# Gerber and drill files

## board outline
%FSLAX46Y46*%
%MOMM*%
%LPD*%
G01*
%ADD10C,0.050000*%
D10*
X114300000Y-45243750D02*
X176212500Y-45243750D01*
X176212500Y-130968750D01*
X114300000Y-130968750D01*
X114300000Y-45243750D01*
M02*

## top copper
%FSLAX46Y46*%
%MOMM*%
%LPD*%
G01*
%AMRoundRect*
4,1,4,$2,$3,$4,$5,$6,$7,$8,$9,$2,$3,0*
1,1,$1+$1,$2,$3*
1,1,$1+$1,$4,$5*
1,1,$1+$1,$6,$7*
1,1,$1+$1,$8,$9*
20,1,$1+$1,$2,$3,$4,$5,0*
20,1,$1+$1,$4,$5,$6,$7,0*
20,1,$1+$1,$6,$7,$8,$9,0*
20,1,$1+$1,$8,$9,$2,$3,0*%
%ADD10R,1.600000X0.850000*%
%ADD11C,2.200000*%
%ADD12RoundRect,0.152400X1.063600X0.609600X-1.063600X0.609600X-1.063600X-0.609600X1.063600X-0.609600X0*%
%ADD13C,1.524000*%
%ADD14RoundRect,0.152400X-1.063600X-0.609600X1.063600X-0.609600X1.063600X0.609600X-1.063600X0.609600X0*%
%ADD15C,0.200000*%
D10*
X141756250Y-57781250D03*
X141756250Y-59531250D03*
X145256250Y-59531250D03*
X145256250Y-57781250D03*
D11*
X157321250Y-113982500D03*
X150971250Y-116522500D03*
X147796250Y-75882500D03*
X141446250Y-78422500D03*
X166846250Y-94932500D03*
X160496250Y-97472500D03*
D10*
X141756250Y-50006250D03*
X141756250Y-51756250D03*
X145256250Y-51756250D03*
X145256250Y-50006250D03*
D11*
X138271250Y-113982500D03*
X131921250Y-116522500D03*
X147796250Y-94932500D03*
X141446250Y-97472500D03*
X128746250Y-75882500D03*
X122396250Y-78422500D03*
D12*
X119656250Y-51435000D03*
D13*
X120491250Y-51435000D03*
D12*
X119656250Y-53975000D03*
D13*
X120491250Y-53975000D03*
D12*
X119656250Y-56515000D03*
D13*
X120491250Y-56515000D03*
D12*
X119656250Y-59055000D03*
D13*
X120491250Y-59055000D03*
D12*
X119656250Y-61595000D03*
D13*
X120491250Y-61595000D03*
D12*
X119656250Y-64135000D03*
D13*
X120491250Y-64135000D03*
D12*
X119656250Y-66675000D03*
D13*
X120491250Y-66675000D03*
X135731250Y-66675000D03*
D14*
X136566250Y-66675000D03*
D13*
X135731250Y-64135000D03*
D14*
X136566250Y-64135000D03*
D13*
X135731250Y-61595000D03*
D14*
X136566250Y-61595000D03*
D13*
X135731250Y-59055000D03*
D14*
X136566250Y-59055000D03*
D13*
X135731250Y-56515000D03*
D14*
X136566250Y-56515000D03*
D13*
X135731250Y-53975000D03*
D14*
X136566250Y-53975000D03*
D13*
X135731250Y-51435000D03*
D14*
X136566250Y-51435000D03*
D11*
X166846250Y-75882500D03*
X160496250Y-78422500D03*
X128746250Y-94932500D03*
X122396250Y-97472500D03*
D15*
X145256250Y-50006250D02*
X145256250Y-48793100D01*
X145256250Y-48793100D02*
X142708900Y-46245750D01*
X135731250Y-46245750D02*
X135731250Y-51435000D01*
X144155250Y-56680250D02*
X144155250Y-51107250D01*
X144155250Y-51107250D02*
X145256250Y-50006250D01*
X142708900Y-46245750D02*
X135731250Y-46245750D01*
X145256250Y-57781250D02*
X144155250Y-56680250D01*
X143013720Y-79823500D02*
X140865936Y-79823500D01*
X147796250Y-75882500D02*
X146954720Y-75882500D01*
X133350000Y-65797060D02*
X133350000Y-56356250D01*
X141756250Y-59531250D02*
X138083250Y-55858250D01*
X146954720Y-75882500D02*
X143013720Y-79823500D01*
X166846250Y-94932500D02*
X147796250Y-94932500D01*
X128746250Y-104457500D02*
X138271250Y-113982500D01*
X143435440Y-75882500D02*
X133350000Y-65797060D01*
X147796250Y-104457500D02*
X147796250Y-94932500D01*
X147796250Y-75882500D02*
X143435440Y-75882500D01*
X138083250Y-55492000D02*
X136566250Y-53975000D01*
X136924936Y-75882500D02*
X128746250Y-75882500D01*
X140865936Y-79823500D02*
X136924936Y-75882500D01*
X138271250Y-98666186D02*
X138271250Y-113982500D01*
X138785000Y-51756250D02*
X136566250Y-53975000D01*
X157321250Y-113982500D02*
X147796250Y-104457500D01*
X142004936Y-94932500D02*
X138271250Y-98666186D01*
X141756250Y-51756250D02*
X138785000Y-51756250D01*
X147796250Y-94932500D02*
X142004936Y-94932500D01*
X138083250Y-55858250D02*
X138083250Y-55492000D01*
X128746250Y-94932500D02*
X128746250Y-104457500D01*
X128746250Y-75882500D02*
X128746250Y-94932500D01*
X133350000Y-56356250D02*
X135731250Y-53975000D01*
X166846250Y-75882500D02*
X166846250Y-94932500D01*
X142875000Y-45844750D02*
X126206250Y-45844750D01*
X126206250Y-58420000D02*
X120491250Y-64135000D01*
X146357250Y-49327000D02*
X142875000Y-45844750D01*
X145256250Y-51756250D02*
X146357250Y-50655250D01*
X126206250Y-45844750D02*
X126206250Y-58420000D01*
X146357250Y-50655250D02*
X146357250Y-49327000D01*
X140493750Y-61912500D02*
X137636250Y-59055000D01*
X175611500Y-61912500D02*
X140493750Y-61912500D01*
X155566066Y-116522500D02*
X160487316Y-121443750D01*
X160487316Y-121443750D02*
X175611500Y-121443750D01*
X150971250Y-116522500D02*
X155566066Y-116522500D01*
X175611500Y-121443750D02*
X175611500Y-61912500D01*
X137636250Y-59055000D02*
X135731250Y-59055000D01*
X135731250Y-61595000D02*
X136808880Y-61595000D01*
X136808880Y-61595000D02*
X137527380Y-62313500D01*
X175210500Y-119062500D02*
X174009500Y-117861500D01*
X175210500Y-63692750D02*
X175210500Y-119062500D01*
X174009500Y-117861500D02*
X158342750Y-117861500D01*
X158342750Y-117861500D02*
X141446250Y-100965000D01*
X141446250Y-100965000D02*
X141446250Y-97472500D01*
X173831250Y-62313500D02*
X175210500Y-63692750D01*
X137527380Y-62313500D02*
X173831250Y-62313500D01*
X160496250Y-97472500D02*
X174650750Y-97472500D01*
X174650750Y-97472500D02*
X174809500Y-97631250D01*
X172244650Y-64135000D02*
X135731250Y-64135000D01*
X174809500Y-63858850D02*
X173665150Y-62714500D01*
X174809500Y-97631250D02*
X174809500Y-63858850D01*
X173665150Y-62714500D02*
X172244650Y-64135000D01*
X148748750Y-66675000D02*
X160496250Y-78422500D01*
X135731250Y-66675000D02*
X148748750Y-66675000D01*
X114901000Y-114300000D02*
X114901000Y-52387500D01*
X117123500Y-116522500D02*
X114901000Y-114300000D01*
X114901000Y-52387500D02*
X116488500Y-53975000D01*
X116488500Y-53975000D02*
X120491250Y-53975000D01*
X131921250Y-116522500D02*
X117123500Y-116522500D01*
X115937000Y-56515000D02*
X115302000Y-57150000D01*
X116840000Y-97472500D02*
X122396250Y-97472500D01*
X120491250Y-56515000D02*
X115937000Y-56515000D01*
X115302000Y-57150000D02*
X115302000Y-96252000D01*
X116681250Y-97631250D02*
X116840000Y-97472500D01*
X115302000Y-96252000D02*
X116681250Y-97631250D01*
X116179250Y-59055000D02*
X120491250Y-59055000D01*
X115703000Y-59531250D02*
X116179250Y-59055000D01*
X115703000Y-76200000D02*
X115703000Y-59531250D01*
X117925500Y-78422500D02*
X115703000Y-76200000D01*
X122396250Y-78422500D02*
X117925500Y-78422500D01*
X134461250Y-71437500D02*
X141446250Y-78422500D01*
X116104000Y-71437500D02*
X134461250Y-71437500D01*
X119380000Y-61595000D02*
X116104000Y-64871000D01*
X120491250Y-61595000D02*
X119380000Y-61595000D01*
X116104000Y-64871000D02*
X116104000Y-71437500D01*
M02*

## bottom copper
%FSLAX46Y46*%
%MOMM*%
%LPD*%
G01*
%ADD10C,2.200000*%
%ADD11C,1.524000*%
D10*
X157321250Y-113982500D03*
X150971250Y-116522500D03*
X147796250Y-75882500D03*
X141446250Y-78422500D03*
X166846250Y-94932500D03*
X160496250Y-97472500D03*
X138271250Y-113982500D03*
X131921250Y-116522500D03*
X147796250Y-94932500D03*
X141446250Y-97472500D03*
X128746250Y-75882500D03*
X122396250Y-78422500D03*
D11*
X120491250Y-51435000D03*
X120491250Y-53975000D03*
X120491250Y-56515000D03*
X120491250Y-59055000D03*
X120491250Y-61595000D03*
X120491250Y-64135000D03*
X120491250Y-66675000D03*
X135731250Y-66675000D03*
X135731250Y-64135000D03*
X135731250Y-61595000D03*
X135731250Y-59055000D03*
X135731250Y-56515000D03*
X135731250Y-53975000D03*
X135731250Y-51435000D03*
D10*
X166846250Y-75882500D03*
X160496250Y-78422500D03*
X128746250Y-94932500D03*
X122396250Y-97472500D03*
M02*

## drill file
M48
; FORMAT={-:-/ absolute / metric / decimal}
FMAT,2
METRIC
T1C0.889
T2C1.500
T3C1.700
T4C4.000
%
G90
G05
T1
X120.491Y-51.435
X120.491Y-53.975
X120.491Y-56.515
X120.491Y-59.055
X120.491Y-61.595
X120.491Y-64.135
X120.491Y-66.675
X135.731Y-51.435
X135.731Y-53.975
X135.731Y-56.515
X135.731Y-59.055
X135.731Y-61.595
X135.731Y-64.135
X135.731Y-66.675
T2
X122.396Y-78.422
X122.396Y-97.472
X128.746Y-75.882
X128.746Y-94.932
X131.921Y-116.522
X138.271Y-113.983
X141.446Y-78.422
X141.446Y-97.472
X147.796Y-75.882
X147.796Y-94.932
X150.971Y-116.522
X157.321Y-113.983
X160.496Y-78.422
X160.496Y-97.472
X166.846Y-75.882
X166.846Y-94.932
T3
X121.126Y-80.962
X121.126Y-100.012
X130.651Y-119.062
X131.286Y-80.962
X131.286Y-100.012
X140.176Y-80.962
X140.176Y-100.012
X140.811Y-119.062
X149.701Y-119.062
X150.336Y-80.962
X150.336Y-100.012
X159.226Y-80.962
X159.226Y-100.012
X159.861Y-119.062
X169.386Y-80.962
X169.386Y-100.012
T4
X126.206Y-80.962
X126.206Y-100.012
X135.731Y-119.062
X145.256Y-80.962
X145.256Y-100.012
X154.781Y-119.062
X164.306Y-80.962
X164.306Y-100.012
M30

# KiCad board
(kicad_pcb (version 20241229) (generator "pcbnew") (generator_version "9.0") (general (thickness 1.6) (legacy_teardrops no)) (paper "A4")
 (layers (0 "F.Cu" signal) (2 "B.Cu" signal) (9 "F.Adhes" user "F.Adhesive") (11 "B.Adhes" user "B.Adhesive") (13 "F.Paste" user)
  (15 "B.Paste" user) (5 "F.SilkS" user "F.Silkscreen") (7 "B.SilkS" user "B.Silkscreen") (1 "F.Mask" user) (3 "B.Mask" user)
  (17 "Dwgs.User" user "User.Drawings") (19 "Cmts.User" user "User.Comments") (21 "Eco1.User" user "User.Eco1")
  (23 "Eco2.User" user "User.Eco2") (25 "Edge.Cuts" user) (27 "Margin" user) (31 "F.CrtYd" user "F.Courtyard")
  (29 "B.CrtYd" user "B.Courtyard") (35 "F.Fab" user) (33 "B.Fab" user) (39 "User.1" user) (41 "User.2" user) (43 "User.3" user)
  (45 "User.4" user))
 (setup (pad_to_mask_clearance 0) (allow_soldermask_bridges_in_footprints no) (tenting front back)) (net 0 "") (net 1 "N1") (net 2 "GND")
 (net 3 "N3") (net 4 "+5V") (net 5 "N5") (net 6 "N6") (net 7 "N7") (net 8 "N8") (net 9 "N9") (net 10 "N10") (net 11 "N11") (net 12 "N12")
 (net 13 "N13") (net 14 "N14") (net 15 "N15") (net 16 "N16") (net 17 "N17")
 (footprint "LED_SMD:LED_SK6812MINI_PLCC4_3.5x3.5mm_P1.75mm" (layer "F.Cu") (at 143.50625 58.65625)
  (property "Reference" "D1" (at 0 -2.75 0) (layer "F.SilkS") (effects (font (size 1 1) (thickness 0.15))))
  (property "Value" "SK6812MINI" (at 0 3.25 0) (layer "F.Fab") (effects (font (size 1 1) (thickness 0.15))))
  (pad "1" smd rect (at -1.75 -0.875) (size 1.6 0.85) (layers "F.Cu" "F.Mask" "F.Paste") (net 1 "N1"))
  (pad "2" smd rect (at -1.75 0.875) (size 1.6 0.85) (layers "F.Cu" "F.Mask" "F.Paste") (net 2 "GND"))
  (pad "3" smd rect (at 1.75 0.875) (size 1.6 0.85) (layers "F.Cu" "F.Mask" "F.Paste") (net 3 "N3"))
  (pad "4" smd rect (at 1.75 -0.875) (size 1.6 0.85) (layers "F.Cu" "F.Mask" "F.Paste") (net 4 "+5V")))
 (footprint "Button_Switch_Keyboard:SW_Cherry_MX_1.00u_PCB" (layer "F.Cu") (at 157.32125 113.9825)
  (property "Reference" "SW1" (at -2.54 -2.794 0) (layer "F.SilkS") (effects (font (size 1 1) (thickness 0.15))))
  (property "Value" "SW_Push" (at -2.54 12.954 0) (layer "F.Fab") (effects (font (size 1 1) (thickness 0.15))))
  (pad "" np_thru_hole circle (at -7.62 5.08) (size 1.7 1.7) (drill 1.7) (layers "*.Cu" "*.Mask"))
  (pad "" np_thru_hole circle (at -2.54 5.08) (size 4 4) (drill 4) (layers "*.Cu" "*.Mask"))
  (pad "" np_thru_hole circle (at 2.54 5.08) (size 1.7 1.7) (drill 1.7) (layers "*.Cu" "*.Mask"))
  (pad "1" thru_hole circle (at 0 0) (size 2.2 2.2) (drill 1.5) (layers "*.Cu" "*.Mask") (remove_unused_layers no) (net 2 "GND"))
  (pad "2" thru_hole circle (at -6.35 2.54) (size 2.2 2.2) (drill 1.5) (layers "*.Cu" "*.Mask") (remove_unused_layers no) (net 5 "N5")))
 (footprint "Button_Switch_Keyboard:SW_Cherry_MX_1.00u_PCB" (layer "F.Cu") (at 147.79625 75.8825)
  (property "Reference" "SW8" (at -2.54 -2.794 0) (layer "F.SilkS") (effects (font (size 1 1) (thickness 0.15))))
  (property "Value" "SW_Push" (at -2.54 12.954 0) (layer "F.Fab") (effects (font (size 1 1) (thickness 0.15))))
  (pad "" np_thru_hole circle (at -7.62 5.08) (size 1.7 1.7) (drill 1.7) (layers "*.Cu" "*.Mask"))
  (pad "" np_thru_hole circle (at -2.54 5.08) (size 4 4) (drill 4) (layers "*.Cu" "*.Mask"))
  (pad "" np_thru_hole circle (at 2.54 5.08) (size 1.7 1.7) (drill 1.7) (layers "*.Cu" "*.Mask"))
  (pad "1" thru_hole circle (at 0 0) (size 2.2 2.2) (drill 1.5) (layers "*.Cu" "*.Mask") (remove_unused_layers no) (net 2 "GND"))
  (pad "2" thru_hole circle (at -6.35 2.54) (size 2.2 2.2) (drill 1.5) (layers "*.Cu" "*.Mask") (remove_unused_layers no) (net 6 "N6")))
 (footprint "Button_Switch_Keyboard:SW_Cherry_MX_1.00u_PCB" (layer "F.Cu") (at 166.84625 94.9325)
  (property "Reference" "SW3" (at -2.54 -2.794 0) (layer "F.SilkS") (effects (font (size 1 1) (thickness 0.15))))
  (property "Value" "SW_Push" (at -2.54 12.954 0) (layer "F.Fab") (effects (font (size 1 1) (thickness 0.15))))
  (pad "" np_thru_hole circle (at -7.62 5.08) (size 1.7 1.7) (drill 1.7) (layers "*.Cu" "*.Mask"))
  (pad "" np_thru_hole circle (at -2.54 5.08) (size 4 4) (drill 4) (layers "*.Cu" "*.Mask"))
  (pad "" np_thru_hole circle (at 2.54 5.08) (size 1.7 1.7) (drill 1.7) (layers "*.Cu" "*.Mask"))
  (pad "1" thru_hole circle (at 0 0) (size 2.2 2.2) (drill 1.5) (layers "*.Cu" "*.Mask") (remove_unused_layers no) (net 2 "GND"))
  (pad "2" thru_hole circle (at -6.35 2.54) (size 2.2 2.2) (drill 1.5) (layers "*.Cu" "*.Mask") (remove_unused_layers no) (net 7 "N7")))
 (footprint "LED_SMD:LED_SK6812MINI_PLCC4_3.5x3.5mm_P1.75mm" (layer "F.Cu") (at 143.50625 50.88125)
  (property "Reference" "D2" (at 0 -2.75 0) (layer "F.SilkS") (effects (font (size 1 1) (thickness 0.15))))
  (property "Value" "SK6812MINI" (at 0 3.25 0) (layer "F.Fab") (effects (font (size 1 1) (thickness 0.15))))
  (pad "1" smd rect (at -1.75 -0.875) (size 1.6 0.85) (layers "F.Cu" "F.Mask" "F.Paste") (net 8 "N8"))
  (pad "2" smd rect (at -1.75 0.875) (size 1.6 0.85) (layers "F.Cu" "F.Mask" "F.Paste") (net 2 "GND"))
  (pad "3" smd rect (at 1.75 0.875) (size 1.6 0.85) (layers "F.Cu" "F.Mask" "F.Paste") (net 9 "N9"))
  (pad "4" smd rect (at 1.75 -0.875) (size 1.6 0.85) (layers "F.Cu" "F.Mask" "F.Paste") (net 4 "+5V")))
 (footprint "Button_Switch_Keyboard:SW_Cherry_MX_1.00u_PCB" (layer "F.Cu") (at 138.27125 113.9825)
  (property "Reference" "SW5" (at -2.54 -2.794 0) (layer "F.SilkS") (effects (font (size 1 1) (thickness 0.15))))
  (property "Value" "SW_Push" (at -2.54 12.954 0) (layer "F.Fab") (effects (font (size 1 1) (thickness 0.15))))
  (pad "" np_thru_hole circle (at -7.62 5.08) (size 1.7 1.7) (drill 1.7) (layers "*.Cu" "*.Mask"))
  (pad "" np_thru_hole circle (at -2.54 5.08) (size 4 4) (drill 4) (layers "*.Cu" "*.Mask"))
  (pad "" np_thru_hole circle (at 2.54 5.08) (size 1.7 1.7) (drill 1.7) (layers "*.Cu" "*.Mask"))
  (pad "1" thru_hole circle (at 0 0) (size 2.2 2.2) (drill 1.5) (layers "*.Cu" "*.Mask") (remove_unused_layers no) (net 2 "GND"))
  (pad "2" thru_hole circle (at -6.35 2.54) (size 2.2 2.2) (drill 1.5) (layers "*.Cu" "*.Mask") (remove_unused_layers no) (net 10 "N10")))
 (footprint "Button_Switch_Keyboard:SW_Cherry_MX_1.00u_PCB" (layer "F.Cu") (at 147.79625 94.9325)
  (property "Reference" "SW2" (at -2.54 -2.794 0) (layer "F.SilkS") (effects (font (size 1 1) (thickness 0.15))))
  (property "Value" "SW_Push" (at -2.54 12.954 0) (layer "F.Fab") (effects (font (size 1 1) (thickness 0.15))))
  (pad "" np_thru_hole circle (at -7.62 5.08) (size 1.7 1.7) (drill 1.7) (layers "*.Cu" "*.Mask"))
  (pad "" np_thru_hole circle (at -2.54 5.08) (size 4 4) (drill 4) (layers "*.Cu" "*.Mask"))
  (pad "" np_thru_hole circle (at 2.54 5.08) (size 1.7 1.7) (drill 1.7) (layers "*.Cu" "*.Mask"))
  (pad "1" thru_hole circle (at 0 0) (size 2.2 2.2) (drill 1.5) (layers "*.Cu" "*.Mask") (remove_unused_layers no) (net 2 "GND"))
  (pad "2" thru_hole circle (at -6.35 2.54) (size 2.2 2.2) (drill 1.5) (layers "*.Cu" "*.Mask") (remove_unused_layers no) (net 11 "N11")))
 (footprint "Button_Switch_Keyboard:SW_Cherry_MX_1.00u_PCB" (layer "F.Cu") (at 128.74625 75.8825)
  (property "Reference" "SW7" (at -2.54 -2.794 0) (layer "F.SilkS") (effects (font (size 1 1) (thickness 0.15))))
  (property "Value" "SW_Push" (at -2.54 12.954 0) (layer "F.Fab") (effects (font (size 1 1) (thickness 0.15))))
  (pad "" np_thru_hole circle (at -7.62 5.08) (size 1.7 1.7) (drill 1.7) (layers "*.Cu" "*.Mask"))
  (pad "" np_thru_hole circle (at -2.54 5.08) (size 4 4) (drill 4) (layers "*.Cu" "*.Mask"))
  (pad "" np_thru_hole circle (at 2.54 5.08) (size 1.7 1.7) (drill 1.7) (layers "*.Cu" "*.Mask"))
  (pad "1" thru_hole circle (at 0 0) (size 2.2 2.2) (drill 1.5) (layers "*.Cu" "*.Mask") (remove_unused_layers no) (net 2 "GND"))
  (pad "2" thru_hole circle (at -6.35 2.54) (size 2.2 2.2) (drill 1.5) (layers "*.Cu" "*.Mask") (remove_unused_layers no) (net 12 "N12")))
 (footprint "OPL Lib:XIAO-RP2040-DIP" (layer "F.Cu") (at 128.11125 59.055)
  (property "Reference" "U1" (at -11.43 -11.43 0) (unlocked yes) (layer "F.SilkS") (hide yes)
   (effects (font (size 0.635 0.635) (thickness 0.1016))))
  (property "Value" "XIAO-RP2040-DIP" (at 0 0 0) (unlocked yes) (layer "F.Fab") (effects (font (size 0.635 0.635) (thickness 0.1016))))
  (pad "1" smd roundrect (at -8.455 -7.62 180) (size 2.432 1.524) (layers "F.Cu" "F.Mask") (roundrect_rratio 0.1) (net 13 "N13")
   (thermal_bridge_angle 45))
  (pad "1" thru_hole circle (at -7.62 -7.62 180) (size 1.524 1.524) (drill 0.889) (layers "*.Cu" "*.Mask") (remove_unused_layers no)
   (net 13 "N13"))
  (pad "2" smd roundrect (at -8.455 -5.08 180) (size 2.432 1.524) (layers "F.Cu" "F.Mask") (roundrect_rratio 0.1) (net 10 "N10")
   (thermal_bridge_angle 45))
  (pad "2" thru_hole circle (at -7.62 -5.08 180) (size 1.524 1.524) (drill 0.889) (layers "*.Cu" "*.Mask") (remove_unused_layers no)
   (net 10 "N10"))
  (pad "3" smd roundrect (at -8.455 -2.54 180) (size 2.432 1.524) (layers "F.Cu" "F.Mask") (roundrect_rratio 0.1) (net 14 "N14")
   (thermal_bridge_angle 45))
  (pad "3" thru_hole circle (at -7.62 -2.54 180) (size 1.524 1.524) (drill 0.889) (layers "*.Cu" "*.Mask") (remove_unused_layers no)
   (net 14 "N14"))
  (pad "4" smd roundrect (at -8.455 0 180) (size 2.432 1.524) (layers "F.Cu" "F.Mask") (roundrect_rratio 0.1) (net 12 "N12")
   (thermal_bridge_angle 45))
  (pad "4" thru_hole circle (at -7.62 0 180) (size 1.524 1.524) (drill 0.889) (layers "*.Cu" "*.Mask") (remove_unused_layers no)
   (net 12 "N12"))
  (pad "5" smd roundrect (at -8.455 2.54 180) (size 2.432 1.524) (layers "F.Cu" "F.Mask") (roundrect_rratio 0.1) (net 6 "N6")
   (thermal_bridge_angle 45))
  (pad "5" thru_hole circle (at -7.62 2.54 180) (size 1.524 1.524) (drill 0.889) (layers "*.Cu" "*.Mask") (remove_unused_layers no)
   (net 6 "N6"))
  (pad "6" smd roundrect (at -8.455 5.08 180) (size 2.432 1.524) (layers "F.Cu" "F.Mask") (roundrect_rratio 0.1) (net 9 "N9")
   (thermal_bridge_angle 45))
  (pad "6" thru_hole circle (at -7.62 5.08 180) (size 1.524 1.524) (drill 0.889) (layers "*.Cu" "*.Mask") (remove_unused_layers no)
   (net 9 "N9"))
  (pad "7" smd roundrect (at -8.455 7.62 180) (size 2.432 1.524) (layers "F.Cu" "F.Mask") (roundrect_rratio 0.1) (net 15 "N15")
   (thermal_bridge_angle 45))
  (pad "7" thru_hole circle (at -7.62 7.62 180) (size 1.524 1.524) (drill 0.889) (layers "*.Cu" "*.Mask") (remove_unused_layers no)
   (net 15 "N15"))
  (pad "8" thru_hole circle (at 7.62 7.62) (size 1.524 1.524) (drill 0.889) (layers "*.Cu" "*.Mask") (remove_unused_layers no)
   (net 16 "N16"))
  (pad "8" smd roundrect (at 8.455 7.62) (size 2.432 1.524) (layers "F.Cu" "F.Mask") (roundrect_rratio 0.1) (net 16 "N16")
   (thermal_bridge_angle 45))
  (pad "9" thru_hole circle (at 7.62 5.08) (size 1.524 1.524) (drill 0.889) (layers "*.Cu" "*.Mask") (remove_unused_layers no) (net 7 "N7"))
  (pad "9" smd roundrect (at 8.455 5.08) (size 2.432 1.524) (layers "F.Cu" "F.Mask") (roundrect_rratio 0.1) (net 7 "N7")
   (thermal_bridge_angle 45))
  (pad "10" thru_hole circle (at 7.62 2.54) (size 1.524 1.524) (drill 0.889) (layers "*.Cu" "*.Mask") (remove_unused_layers no)
   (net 11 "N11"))
  (pad "10" smd roundrect (at 8.455 2.54) (size 2.432 1.524) (layers "F.Cu" "F.Mask") (roundrect_rratio 0.1) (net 11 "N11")
   (thermal_bridge_angle 45))
  (pad "11" thru_hole circle (at 7.62 0) (size 1.524 1.524) (drill 0.889) (layers "*.Cu" "*.Mask") (remove_unused_layers no) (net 5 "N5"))
  (pad "11" smd roundrect (at 8.455 0) (size 2.432 1.524) (layers "F.Cu" "F.Mask") (roundrect_rratio 0.1) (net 5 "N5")
   (thermal_bridge_angle 45))
  (pad "12" thru_hole circle (at 7.62 -2.54) (size 1.524 1.524) (drill 0.889) (layers "*.Cu" "*.Mask") (remove_unused_layers no)
   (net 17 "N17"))
  (pad "12" smd roundrect (at 8.455 -2.54) (size 2.432 1.524) (layers "F.Cu" "F.Mask") (roundrect_rratio 0.1) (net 17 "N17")
   (thermal_bridge_angle 45))
  (pad "13" thru_hole circle (at 7.62 -5.08) (size 1.524 1.524) (drill 0.889) (layers "*.Cu" "*.Mask") (remove_unused_layers no)
   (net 2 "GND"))
  (pad "13" smd roundrect (at 8.455 -5.08) (size 2.432 1.524) (layers "F.Cu" "F.Mask") (roundrect_rratio 0.1) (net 2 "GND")
   (thermal_bridge_angle 45))
  (pad "14" thru_hole circle (at 7.62 -7.62) (size 1.524 1.524) (drill 0.889) (layers "*.Cu" "*.Mask") (remove_unused_layers no)
   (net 4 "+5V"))
  (pad "14" smd roundrect (at 8.455 -7.62) (size 2.432 1.524) (layers "F.Cu" "F.Mask") (roundrect_rratio 0.1) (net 4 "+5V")
   (thermal_bridge_angle 45)))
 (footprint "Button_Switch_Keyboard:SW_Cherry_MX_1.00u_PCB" (layer "F.Cu") (at 166.84625 75.8825)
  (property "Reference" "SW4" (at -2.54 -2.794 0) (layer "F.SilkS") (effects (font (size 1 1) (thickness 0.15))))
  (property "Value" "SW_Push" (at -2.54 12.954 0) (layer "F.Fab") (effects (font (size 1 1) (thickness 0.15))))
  (pad "" np_thru_hole circle (at -7.62 5.08) (size 1.7 1.7) (drill 1.7) (layers "*.Cu" "*.Mask"))
  (pad "" np_thru_hole circle (at -2.54 5.08) (size 4 4) (drill 4) (layers "*.Cu" "*.Mask"))
  (pad "" np_thru_hole circle (at 2.54 5.08) (size 1.7 1.7) (drill 1.7) (layers "*.Cu" "*.Mask"))
  (pad "1" thru_hole circle (at 0 0) (size 2.2 2.2) (drill 1.5) (layers "*.Cu" "*.Mask") (remove_unused_layers no) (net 2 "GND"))
  (pad "2" thru_hole circle (at -6.35 2.54) (size 2.2 2.2) (drill 1.5) (layers "*.Cu" "*.Mask") (remove_unused_layers no) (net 16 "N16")))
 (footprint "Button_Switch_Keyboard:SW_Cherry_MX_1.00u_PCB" (layer "F.Cu") (at 128.74625 94.9325)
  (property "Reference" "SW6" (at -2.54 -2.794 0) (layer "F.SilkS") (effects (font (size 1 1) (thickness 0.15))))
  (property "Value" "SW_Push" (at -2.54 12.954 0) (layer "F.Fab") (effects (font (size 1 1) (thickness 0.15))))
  (pad "" np_thru_hole circle (at -7.62 5.08) (size 1.7 1.7) (drill 1.7) (layers "*.Cu" "*.Mask"))
  (pad "" np_thru_hole circle (at -2.54 5.08) (size 4 4) (drill 4) (layers "*.Cu" "*.Mask"))
  (pad "" np_thru_hole circle (at 2.54 5.08) (size 1.7 1.7) (drill 1.7) (layers "*.Cu" "*.Mask"))
  (pad "1" thru_hole circle (at 0 0) (size 2.2 2.2) (drill 1.5) (layers "*.Cu" "*.Mask") (remove_unused_layers no) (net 2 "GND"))
  (pad "2" thru_hole circle (at -6.35 2.54) (size 2.2 2.2) (drill 1.5) (layers "*.Cu" "*.Mask") (remove_unused_layers no) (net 14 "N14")))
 (gr_rect (start 114.3 45.24375) (end 176.2125 130.96875) (stroke (width 0.05) (type default)) (fill no) (layer "Edge.Cuts"))
 (segment (start 145.25625 50.00625) (end 145.25625 48.7931) (width 0.2) (layer "F.Cu") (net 4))
 (segment (start 145.25625 48.7931) (end 142.7089 46.24575) (width 0.2) (layer "F.Cu") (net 4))
 (segment (start 135.73125 46.24575) (end 135.73125 51.435) (width 0.2) (layer "F.Cu") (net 4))
 (segment (start 144.15525 56.68025) (end 144.15525 51.10725) (width 0.2) (layer "F.Cu") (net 4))
 (segment (start 144.15525 51.10725) (end 145.25625 50.00625) (width 0.2) (layer "F.Cu") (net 4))
 (segment (start 142.7089 46.24575) (end 135.73125 46.24575) (width 0.2) (layer "F.Cu") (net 4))
 (segment (start 145.25625 57.78125) (end 144.15525 56.68025) (width 0.2) (layer "F.Cu") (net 4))
 (segment (start 143.01372 79.8235) (end 140.865936 79.8235) (width 0.2) (layer "F.Cu") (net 2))
 (segment (start 147.79625 75.8825) (end 146.95472 75.8825) (width 0.2) (layer "F.Cu") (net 2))
 (segment (start 133.35 65.79706) (end 133.35 56.35625) (width 0.2) (layer "F.Cu") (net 2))
 (segment (start 141.75625 59.53125) (end 138.08325 55.85825) (width 0.2) (layer "F.Cu") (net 2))
 (segment (start 146.95472 75.8825) (end 143.01372 79.8235) (width 0.2) (layer "F.Cu") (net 2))
 (segment (start 166.84625 94.9325) (end 147.79625 94.9325) (width 0.2) (layer "F.Cu") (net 2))
 (segment (start 128.74625 104.4575) (end 138.27125 113.9825) (width 0.2) (layer "F.Cu") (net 2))
 (segment (start 143.43544 75.8825) (end 133.35 65.79706) (width 0.2) (layer "F.Cu") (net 2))
 (segment (start 147.79625 104.4575) (end 147.79625 94.9325) (width 0.2) (layer "F.Cu") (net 2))
 (segment (start 147.79625 75.8825) (end 143.43544 75.8825) (width 0.2) (layer "F.Cu") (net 2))
 (segment (start 138.08325 55.492) (end 136.56625 53.975) (width 0.2) (layer "F.Cu") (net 2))
 (segment (start 136.924936 75.8825) (end 128.74625 75.8825) (width 0.2) (layer "F.Cu") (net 2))
 (segment (start 140.865936 79.8235) (end 136.924936 75.8825) (width 0.2) (layer "F.Cu") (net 2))
 (segment (start 138.27125 98.666186) (end 138.27125 113.9825) (width 0.2) (layer "F.Cu") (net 2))
 (segment (start 138.785 51.75625) (end 136.56625 53.975) (width 0.2) (layer "F.Cu") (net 2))
 (segment (start 157.32125 113.9825) (end 147.79625 104.4575) (width 0.2) (layer "F.Cu") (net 2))
 (segment (start 142.004936 94.9325) (end 138.27125 98.666186) (width 0.2) (layer "F.Cu") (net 2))
 (segment (start 141.75625 51.75625) (end 138.785 51.75625) (width 0.2) (layer "F.Cu") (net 2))
 (segment (start 147.79625 94.9325) (end 142.004936 94.9325) (width 0.2) (layer "F.Cu") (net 2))
 (segment (start 138.08325 55.85825) (end 138.08325 55.492) (width 0.2) (layer "F.Cu") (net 2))
 (segment (start 128.74625 94.9325) (end 128.74625 104.4575) (width 0.2) (layer "F.Cu") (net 2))
 (segment (start 128.74625 75.8825) (end 128.74625 94.9325) (width 0.2) (layer "F.Cu") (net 2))
 (segment (start 133.35 56.35625) (end 135.73125 53.975) (width 0.2) (layer "F.Cu") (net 2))
 (segment (start 166.84625 75.8825) (end 166.84625 94.9325) (width 0.2) (layer "F.Cu") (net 2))
 (segment (start 142.875 45.84475) (end 126.20625 45.84475) (width 0.2) (layer "F.Cu") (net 9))
 (segment (start 126.20625 58.42) (end 120.49125 64.135) (width 0.2) (layer "F.Cu") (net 9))
 (segment (start 146.35725 49.327) (end 142.875 45.84475) (width 0.2) (layer "F.Cu") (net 9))
 (segment (start 145.25625 51.75625) (end 146.35725 50.65525) (width 0.2) (layer "F.Cu") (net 9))
 (segment (start 126.20625 45.84475) (end 126.20625 58.42) (width 0.2) (layer "F.Cu") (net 9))
 (segment (start 146.35725 50.65525) (end 146.35725 49.327) (width 0.2) (layer "F.Cu") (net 9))
 (segment (start 140.49375 61.9125) (end 137.63625 59.055) (width 0.2) (layer "F.Cu") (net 5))
 (segment (start 175.6115 61.9125) (end 140.49375 61.9125) (width 0.2) (layer "F.Cu") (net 5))
 (segment (start 155.566066 116.5225) (end 160.487316 121.44375) (width 0.2) (layer "F.Cu") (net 5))
 (segment (start 160.487316 121.44375) (end 175.6115 121.44375) (width 0.2) (layer "F.Cu") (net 5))
 (segment (start 150.97125 116.5225) (end 155.566066 116.5225) (width 0.2) (layer "F.Cu") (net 5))
 (segment (start 175.6115 121.44375) (end 175.6115 61.9125) (width 0.2) (layer "F.Cu") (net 5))
 (segment (start 137.63625 59.055) (end 135.73125 59.055) (width 0.2) (layer "F.Cu") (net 5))
 (segment (start 135.73125 61.595) (end 136.80888 61.595) (width 0.2) (layer "F.Cu") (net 11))
 (segment (start 136.80888 61.595) (end 137.52738 62.3135) (width 0.2) (layer "F.Cu") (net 11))
 (segment (start 175.2105 119.0625) (end 174.0095 117.8615) (width 0.2) (layer "F.Cu") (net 11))
 (segment (start 175.2105 63.69275) (end 175.2105 119.0625) (width 0.2) (layer "F.Cu") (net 11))
 (segment (start 174.0095 117.8615) (end 158.34275 117.8615) (width 0.2) (layer "F.Cu") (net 11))
 (segment (start 158.34275 117.8615) (end 141.44625 100.965) (width 0.2) (layer "F.Cu") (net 11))
 (segment (start 141.44625 100.965) (end 141.44625 97.4725) (width 0.2) (layer "F.Cu") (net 11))
 (segment (start 173.83125 62.3135) (end 175.2105 63.69275) (width 0.2) (layer "F.Cu") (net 11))
 (segment (start 137.52738 62.3135) (end 173.83125 62.3135) (width 0.2) (layer "F.Cu") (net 11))
 (segment (start 160.49625 97.4725) (end 174.65075 97.4725) (width 0.2) (layer "F.Cu") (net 7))
 (segment (start 174.65075 97.4725) (end 174.8095 97.63125) (width 0.2) (layer "F.Cu") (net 7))
 (segment (start 172.24465 64.135) (end 135.73125 64.135) (width 0.2) (layer "F.Cu") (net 7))
 (segment (start 174.8095 63.85885) (end 173.66515 62.7145) (width 0.2) (layer "F.Cu") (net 7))
 (segment (start 174.8095 97.63125) (end 174.8095 63.85885) (width 0.2) (layer "F.Cu") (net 7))
 (segment (start 173.66515 62.7145) (end 172.24465 64.135) (width 0.2) (layer "F.Cu") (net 7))
 (segment (start 148.74875 66.675) (end 160.49625 78.4225) (width 0.2) (layer "F.Cu") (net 16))
 (segment (start 135.73125 66.675) (end 148.74875 66.675) (width 0.2) (layer "F.Cu") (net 16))
 (segment (start 114.901 114.3) (end 114.901 52.3875) (width 0.2) (layer "F.Cu") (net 10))
 (segment (start 117.1235 116.5225) (end 114.901 114.3) (width 0.2) (layer "F.Cu") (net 10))
 (segment (start 114.901 52.3875) (end 116.4885 53.975) (width 0.2) (layer "F.Cu") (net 10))
 (segment (start 116.4885 53.975) (end 120.49125 53.975) (width 0.2) (layer "F.Cu") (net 10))
 (segment (start 131.92125 116.5225) (end 117.1235 116.5225) (width 0.2) (layer "F.Cu") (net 10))
 (segment (start 115.937 56.515) (end 115.302 57.15) (width 0.2) (layer "F.Cu") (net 14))
 (segment (start 116.84 97.4725) (end 122.39625 97.4725) (width 0.2) (layer "F.Cu") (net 14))
 (segment (start 120.49125 56.515) (end 115.937 56.515) (width 0.2) (layer "F.Cu") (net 14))
 (segment (start 115.302 57.15) (end 115.302 96.252) (width 0.2) (layer "F.Cu") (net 14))
 (segment (start 116.68125 97.63125) (end 116.84 97.4725) (width 0.2) (layer "F.Cu") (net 14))
 (segment (start 115.302 96.252) (end 116.68125 97.63125) (width 0.2) (layer "F.Cu") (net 14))
 (segment (start 116.17925 59.055) (end 120.49125 59.055) (width 0.2) (layer "F.Cu") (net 12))
 (segment (start 115.703 59.53125) (end 116.17925 59.055) (width 0.2) (layer "F.Cu") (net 12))
 (segment (start 115.703 76.2) (end 115.703 59.53125) (width 0.2) (layer "F.Cu") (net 12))
 (segment (start 117.9255 78.4225) (end 115.703 76.2) (width 0.2) (layer "F.Cu") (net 12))
 (segment (start 122.39625 78.4225) (end 117.9255 78.4225) (width 0.2) (layer "F.Cu") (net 12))
 (segment (start 134.46125 71.4375) (end 141.44625 78.4225) (width 0.2) (layer "F.Cu") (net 6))
 (segment (start 116.104 71.4375) (end 134.46125 71.4375) (width 0.2) (layer "F.Cu") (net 6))
 (segment (start 119.38 61.595) (end 116.104 64.871) (width 0.2) (layer "F.Cu") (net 6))
 (segment (start 120.49125 61.595) (end 119.38 61.595) (width 0.2) (layer "F.Cu") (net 6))
 (segment (start 116.104 64.871) (end 116.104 71.4375) (width 0.2) (layer "F.Cu") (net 6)))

